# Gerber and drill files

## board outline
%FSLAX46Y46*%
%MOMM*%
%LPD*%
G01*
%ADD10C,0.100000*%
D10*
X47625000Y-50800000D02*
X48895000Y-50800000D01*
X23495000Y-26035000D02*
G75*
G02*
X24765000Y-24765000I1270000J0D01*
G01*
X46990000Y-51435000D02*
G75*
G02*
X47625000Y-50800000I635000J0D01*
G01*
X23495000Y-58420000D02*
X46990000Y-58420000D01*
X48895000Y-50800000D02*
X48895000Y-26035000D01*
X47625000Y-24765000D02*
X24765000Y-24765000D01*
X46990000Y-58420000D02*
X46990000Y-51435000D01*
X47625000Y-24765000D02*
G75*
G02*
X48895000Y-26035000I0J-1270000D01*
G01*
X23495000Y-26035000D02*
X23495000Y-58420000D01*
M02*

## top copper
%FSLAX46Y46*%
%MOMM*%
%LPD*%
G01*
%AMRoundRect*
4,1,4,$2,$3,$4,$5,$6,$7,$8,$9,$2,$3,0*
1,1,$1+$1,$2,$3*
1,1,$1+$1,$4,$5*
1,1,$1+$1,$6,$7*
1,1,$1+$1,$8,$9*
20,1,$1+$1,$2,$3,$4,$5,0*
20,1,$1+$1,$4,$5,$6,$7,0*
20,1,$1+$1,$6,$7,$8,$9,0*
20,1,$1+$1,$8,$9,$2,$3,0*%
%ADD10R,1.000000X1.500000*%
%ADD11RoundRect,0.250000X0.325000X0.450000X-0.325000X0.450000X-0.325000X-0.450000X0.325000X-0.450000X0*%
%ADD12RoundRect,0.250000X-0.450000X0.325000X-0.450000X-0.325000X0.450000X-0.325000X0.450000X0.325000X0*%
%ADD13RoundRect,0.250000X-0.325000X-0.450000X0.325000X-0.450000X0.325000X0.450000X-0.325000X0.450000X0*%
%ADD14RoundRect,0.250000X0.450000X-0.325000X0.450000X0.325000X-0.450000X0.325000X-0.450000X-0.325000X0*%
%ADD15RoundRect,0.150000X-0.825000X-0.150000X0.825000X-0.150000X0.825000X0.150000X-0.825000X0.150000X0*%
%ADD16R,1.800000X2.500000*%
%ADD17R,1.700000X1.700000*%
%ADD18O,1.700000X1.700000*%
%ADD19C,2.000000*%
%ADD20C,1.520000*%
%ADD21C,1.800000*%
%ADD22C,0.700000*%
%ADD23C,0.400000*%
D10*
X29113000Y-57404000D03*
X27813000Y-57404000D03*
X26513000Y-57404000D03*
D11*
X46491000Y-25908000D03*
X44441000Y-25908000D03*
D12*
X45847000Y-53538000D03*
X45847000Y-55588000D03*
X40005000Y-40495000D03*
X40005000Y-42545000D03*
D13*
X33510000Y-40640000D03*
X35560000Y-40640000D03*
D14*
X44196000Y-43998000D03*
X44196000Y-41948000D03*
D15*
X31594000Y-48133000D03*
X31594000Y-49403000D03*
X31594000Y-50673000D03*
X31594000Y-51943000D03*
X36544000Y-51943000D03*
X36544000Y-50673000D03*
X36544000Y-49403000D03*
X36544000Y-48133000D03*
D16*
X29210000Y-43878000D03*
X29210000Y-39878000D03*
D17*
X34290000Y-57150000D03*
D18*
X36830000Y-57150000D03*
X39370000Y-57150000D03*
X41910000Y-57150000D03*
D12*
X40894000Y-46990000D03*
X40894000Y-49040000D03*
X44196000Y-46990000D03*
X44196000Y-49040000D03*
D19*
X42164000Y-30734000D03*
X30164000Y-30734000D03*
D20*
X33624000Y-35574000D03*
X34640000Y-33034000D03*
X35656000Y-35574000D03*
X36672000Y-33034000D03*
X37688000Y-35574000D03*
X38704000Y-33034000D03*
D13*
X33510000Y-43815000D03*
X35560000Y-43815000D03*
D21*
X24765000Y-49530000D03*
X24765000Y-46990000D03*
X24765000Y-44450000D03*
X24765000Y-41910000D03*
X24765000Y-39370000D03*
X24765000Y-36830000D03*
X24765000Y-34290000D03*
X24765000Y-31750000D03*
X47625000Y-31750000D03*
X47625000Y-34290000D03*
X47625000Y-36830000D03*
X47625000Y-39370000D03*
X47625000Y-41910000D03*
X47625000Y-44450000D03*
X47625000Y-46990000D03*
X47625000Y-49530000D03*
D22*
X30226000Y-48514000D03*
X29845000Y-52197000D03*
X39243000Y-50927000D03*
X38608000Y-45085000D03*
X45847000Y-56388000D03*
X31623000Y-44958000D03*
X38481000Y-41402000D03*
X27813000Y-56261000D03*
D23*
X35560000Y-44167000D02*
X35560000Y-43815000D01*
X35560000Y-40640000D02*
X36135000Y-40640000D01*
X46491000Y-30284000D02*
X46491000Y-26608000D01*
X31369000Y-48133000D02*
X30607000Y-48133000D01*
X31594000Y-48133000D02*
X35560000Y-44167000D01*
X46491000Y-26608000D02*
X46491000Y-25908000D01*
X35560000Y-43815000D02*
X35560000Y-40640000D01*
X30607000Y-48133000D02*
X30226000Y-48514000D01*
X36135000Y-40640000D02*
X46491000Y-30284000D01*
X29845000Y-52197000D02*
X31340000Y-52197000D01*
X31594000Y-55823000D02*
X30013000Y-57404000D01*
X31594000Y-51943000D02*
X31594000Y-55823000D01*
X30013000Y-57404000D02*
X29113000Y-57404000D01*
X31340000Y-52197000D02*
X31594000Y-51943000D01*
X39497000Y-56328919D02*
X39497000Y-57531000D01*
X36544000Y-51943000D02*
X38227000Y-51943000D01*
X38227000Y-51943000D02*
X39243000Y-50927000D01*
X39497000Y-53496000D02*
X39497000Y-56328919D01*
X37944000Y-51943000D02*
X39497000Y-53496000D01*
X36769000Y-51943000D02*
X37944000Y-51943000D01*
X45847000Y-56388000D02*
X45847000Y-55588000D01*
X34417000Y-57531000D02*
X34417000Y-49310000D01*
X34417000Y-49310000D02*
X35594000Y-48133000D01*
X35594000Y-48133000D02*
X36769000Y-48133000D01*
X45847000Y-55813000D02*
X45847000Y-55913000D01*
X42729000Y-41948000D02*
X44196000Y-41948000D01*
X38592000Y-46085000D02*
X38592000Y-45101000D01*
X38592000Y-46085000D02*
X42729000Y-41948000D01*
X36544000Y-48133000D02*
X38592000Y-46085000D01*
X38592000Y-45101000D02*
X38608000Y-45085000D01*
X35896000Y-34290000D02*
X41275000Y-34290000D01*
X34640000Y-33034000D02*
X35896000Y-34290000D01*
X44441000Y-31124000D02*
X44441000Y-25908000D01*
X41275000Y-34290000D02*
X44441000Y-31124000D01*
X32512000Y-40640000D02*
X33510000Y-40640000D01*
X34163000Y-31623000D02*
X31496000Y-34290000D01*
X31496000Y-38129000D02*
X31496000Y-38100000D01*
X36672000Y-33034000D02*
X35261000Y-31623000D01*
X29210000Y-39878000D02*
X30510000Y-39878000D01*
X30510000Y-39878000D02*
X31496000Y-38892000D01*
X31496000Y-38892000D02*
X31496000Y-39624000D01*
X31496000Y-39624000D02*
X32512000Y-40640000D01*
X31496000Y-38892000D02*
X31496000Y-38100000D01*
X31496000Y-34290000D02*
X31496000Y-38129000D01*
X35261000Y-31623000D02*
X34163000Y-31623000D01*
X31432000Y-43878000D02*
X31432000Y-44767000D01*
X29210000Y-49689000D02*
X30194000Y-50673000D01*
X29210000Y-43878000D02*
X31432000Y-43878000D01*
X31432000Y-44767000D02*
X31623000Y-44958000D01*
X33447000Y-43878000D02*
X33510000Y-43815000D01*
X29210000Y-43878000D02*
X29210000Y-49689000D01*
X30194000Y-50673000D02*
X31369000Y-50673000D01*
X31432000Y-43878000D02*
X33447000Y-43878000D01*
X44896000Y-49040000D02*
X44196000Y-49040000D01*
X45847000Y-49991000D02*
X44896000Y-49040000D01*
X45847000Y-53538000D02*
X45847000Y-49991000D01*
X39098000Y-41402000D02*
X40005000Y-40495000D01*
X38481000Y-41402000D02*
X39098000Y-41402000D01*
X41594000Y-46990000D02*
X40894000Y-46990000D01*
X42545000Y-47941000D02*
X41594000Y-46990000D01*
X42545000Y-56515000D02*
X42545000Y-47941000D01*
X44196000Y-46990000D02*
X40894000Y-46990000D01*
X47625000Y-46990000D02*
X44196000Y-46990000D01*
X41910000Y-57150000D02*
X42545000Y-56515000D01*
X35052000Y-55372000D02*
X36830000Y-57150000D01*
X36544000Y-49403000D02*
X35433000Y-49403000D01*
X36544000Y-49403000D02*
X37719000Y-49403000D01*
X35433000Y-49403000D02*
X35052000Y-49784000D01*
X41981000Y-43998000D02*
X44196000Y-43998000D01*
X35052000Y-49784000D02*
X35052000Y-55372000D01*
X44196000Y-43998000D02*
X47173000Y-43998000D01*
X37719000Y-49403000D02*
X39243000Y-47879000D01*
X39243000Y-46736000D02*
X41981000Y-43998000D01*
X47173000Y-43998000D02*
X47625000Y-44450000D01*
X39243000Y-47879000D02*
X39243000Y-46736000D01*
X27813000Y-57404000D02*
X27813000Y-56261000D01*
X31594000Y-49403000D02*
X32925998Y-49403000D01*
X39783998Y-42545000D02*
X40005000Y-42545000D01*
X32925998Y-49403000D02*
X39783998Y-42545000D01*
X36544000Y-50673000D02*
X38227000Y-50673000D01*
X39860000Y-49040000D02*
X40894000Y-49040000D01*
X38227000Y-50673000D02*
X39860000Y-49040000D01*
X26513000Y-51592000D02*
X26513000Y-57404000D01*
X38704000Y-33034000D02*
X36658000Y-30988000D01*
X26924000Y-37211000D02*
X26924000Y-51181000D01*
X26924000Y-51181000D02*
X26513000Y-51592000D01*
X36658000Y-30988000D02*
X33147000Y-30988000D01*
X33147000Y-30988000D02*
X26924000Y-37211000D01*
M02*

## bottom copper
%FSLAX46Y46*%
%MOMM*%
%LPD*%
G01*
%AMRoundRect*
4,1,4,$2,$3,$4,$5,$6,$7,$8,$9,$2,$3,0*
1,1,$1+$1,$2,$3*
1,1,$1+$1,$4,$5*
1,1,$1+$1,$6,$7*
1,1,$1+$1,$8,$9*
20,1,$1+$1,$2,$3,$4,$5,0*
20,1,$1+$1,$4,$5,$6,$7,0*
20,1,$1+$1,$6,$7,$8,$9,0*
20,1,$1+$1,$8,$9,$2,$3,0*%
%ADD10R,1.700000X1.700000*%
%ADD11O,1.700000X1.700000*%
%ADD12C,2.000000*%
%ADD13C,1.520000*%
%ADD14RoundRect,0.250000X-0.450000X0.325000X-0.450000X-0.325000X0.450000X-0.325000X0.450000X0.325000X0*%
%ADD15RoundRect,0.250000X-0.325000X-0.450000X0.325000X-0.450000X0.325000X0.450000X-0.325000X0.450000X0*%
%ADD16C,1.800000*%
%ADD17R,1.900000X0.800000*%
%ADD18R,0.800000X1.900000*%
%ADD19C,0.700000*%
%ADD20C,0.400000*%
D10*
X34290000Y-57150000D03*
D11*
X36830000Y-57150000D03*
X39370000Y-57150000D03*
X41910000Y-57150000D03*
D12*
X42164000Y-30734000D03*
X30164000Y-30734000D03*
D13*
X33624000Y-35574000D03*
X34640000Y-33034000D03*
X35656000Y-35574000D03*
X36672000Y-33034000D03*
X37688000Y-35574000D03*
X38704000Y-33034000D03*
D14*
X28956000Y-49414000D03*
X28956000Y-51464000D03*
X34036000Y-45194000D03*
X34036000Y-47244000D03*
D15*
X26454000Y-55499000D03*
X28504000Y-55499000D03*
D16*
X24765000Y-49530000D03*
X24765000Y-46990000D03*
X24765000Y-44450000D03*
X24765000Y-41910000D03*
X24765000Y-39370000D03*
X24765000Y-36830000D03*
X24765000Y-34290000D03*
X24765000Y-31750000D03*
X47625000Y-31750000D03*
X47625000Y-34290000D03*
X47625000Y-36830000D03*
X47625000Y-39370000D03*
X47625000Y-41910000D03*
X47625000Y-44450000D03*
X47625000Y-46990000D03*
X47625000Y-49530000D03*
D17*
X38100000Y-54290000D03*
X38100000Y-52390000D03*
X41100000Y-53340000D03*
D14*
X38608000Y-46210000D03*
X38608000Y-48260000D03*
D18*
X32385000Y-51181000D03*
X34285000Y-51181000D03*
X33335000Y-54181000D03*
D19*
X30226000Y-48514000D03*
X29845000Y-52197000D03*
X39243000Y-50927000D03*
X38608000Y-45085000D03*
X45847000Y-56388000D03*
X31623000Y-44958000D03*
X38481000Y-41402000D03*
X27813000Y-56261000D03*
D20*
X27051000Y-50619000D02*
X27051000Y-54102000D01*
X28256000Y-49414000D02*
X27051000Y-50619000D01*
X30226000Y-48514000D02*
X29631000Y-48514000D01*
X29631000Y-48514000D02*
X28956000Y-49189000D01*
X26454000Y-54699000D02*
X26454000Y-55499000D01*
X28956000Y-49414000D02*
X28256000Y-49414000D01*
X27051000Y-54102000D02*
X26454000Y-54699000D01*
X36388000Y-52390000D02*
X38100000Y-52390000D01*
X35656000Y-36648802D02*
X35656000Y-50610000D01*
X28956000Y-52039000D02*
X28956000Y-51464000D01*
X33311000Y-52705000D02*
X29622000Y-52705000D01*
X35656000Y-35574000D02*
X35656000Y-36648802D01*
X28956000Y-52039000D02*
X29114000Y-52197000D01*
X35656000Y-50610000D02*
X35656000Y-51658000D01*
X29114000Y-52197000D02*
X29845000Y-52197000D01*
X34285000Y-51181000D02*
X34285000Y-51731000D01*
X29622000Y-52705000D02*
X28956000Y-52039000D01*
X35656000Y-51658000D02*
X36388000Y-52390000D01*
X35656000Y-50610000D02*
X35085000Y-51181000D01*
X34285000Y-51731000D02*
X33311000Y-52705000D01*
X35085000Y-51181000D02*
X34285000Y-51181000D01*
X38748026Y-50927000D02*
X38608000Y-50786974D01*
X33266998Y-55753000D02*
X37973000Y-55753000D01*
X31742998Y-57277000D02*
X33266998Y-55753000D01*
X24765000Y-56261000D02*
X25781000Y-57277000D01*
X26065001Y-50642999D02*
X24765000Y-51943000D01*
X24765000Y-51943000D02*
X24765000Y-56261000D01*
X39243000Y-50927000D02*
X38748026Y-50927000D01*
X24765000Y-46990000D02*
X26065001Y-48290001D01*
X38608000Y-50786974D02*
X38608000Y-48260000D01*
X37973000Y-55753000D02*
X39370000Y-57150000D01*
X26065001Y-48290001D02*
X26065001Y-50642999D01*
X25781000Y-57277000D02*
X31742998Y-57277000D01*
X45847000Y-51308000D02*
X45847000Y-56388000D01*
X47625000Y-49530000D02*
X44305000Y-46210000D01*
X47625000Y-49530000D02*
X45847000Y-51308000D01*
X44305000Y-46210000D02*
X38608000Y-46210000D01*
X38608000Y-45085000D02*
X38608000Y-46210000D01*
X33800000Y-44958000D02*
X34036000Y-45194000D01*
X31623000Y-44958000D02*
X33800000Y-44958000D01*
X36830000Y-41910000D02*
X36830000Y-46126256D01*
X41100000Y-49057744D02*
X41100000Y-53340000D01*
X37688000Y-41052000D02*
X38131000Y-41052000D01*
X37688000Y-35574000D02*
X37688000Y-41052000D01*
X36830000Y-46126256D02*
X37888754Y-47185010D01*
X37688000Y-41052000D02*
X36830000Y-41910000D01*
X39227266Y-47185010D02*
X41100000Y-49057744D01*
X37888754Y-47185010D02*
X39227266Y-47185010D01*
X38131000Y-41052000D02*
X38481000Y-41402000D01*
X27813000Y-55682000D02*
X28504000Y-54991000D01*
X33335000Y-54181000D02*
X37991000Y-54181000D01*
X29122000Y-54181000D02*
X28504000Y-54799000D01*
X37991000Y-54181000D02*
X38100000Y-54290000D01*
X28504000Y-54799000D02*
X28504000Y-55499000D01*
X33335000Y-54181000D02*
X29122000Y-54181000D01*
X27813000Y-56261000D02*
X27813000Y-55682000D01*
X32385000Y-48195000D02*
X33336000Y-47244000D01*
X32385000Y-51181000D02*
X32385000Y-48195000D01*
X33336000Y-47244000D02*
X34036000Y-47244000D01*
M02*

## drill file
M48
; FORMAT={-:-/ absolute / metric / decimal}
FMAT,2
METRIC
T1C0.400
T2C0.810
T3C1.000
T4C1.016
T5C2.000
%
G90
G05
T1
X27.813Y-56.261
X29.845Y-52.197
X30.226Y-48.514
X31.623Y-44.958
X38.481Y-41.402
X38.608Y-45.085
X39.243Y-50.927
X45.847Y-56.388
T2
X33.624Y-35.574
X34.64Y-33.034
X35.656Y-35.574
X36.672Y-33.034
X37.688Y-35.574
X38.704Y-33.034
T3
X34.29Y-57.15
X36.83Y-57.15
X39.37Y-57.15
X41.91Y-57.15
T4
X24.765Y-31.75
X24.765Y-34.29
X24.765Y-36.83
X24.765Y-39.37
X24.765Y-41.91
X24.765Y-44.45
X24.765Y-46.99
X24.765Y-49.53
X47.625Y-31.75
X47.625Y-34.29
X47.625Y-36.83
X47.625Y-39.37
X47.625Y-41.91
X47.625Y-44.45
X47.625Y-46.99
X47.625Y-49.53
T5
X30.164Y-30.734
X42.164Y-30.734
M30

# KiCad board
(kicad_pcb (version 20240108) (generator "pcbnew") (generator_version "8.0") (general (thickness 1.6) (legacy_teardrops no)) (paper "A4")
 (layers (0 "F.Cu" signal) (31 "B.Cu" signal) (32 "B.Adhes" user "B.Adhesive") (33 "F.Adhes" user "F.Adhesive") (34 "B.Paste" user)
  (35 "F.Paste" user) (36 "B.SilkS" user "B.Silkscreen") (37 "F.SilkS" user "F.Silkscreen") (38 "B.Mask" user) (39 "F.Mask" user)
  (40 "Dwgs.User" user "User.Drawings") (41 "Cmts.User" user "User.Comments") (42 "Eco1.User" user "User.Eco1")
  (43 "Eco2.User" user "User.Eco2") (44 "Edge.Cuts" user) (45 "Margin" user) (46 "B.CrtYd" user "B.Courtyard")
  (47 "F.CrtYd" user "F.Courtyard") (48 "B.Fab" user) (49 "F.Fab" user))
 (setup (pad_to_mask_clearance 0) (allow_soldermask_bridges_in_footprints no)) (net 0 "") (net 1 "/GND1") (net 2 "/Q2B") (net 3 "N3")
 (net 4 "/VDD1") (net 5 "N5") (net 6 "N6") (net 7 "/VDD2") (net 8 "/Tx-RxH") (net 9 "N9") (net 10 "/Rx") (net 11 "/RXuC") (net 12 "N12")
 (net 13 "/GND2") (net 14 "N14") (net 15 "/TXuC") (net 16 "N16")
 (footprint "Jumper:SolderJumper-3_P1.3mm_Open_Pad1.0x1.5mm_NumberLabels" (layer "F.Cu") (at 27.813 57.404 180)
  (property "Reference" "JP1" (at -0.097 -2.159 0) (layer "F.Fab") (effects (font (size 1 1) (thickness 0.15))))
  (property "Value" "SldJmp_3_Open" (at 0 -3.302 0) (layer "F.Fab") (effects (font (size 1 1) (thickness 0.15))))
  (pad "1" smd rect (at -1.3 0 180) (size 1 1.5) (layers "F.Cu" "F.Mask") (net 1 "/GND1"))
  (pad "2" smd rect (at 0 0 180) (size 1 1.5) (layers "F.Cu" "F.Mask") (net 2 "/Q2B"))
  (pad "3" smd rect (at 1.3 0 180) (size 1 1.5) (layers "F.Cu" "F.Mask") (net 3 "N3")))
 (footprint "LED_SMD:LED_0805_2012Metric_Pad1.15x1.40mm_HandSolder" (layer "F.Cu") (at 45.466 25.908 180)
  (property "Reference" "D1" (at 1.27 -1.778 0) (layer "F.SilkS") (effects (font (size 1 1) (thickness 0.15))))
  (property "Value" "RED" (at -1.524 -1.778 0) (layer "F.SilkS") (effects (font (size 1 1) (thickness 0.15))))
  (pad "1" smd roundrect (at -1.025 0 180) (size 1.15 1.4) (layers "F.Cu" "F.Paste" "F.Mask") (roundrect_rratio 0.217391) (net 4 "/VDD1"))
  (pad "2" smd roundrect (at 1.025 0 180) (size 1.15 1.4) (layers "F.Cu" "F.Paste" "F.Mask") (roundrect_rratio 0.217391) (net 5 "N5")))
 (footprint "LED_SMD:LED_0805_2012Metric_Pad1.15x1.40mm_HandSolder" (layer "F.Cu") (at 45.847 54.563 -90)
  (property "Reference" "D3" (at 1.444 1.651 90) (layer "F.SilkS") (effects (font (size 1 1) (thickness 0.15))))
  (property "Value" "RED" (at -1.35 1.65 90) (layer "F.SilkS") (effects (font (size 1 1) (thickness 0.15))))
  (pad "1" smd roundrect (at -1.025 0 270) (size 1.15 1.4) (layers "F.Cu" "F.Paste" "F.Mask") (roundrect_rratio 0.217391) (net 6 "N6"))
  (pad "2" smd roundrect (at 1.025 0 270) (size 1.15 1.4) (layers "F.Cu" "F.Paste" "F.Mask") (roundrect_rratio 0.217391) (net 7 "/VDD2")))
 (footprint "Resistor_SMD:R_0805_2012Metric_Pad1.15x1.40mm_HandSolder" (layer "F.Cu") (at 40.005 41.52 -90)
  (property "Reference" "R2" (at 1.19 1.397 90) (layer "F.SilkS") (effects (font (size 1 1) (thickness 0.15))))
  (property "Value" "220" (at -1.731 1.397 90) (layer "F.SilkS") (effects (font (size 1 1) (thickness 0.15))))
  (pad "1" smd roundrect (at -1.025 0 270) (size 1.15 1.4) (layers "F.Cu" "F.Paste" "F.Mask") (roundrect_rratio 0.217391) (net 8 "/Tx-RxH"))
  (pad "2" smd roundrect (at 1.025 0 270) (size 1.15 1.4) (layers "F.Cu" "F.Paste" "F.Mask") (roundrect_rratio 0.217391) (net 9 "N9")))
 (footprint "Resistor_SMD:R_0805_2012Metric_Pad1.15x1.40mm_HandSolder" (layer "F.Cu") (at 34.535 40.64)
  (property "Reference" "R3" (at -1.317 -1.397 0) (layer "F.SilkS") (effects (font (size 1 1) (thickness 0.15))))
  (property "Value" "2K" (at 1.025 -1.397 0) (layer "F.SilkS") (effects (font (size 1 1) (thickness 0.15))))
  (pad "1" smd roundrect (at -1.025 0) (size 1.15 1.4) (layers "F.Cu" "F.Paste" "F.Mask") (roundrect_rratio 0.217391) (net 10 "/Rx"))
  (pad "2" smd roundrect (at 1.025 0) (size 1.15 1.4) (layers "F.Cu" "F.Paste" "F.Mask") (roundrect_rratio 0.217391) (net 4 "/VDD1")))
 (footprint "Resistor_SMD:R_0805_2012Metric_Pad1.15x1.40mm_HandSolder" (layer "F.Cu") (at 44.196 42.973 90)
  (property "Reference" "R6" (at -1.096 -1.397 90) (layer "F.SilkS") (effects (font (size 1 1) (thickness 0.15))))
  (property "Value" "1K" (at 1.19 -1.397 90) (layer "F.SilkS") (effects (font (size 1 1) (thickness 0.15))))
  (pad "1" smd roundrect (at -1.025 0 90) (size 1.15 1.4) (layers "F.Cu" "F.Paste" "F.Mask") (roundrect_rratio 0.217391) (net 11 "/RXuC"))
  (pad "2" smd roundrect (at 1.025 0 90) (size 1.15 1.4) (layers "F.Cu" "F.Paste" "F.Mask") (roundrect_rratio 0.217391) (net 7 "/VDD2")))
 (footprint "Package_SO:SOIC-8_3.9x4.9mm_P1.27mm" (layer "F.Cu") (at 34.069 50.038)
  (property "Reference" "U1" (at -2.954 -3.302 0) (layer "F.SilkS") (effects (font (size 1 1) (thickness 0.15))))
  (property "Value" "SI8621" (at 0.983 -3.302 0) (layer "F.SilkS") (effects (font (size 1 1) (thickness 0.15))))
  (pad "1" smd roundrect (at -2.475 -1.905) (size 1.95 0.6) (layers "F.Cu" "F.Paste" "F.Mask") (roundrect_rratio 0.25) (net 4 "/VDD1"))
  (pad "2" smd roundrect (at -2.475 -0.635) (size 1.95 0.6) (layers "F.Cu" "F.Paste" "F.Mask") (roundrect_rratio 0.25) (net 9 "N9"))
  (pad "3" smd roundrect (at -2.475 0.635) (size 1.95 0.6) (layers "F.Cu" "F.Paste" "F.Mask") (roundrect_rratio 0.25) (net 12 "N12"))
  (pad "4" smd roundrect (at -2.475 1.905) (size 1.95 0.6) (layers "F.Cu" "F.Paste" "F.Mask") (roundrect_rratio 0.25) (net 1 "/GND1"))
  (pad "5" smd roundrect (at 2.475 1.905) (size 1.95 0.6) (layers "F.Cu" "F.Paste" "F.Mask") (roundrect_rratio 0.25) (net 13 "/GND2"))
  (pad "6" smd roundrect (at 2.475 0.635) (size 1.95 0.6) (layers "F.Cu" "F.Paste" "F.Mask") (roundrect_rratio 0.25) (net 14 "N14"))
  (pad "7" smd roundrect (at 2.475 -0.635) (size 1.95 0.6) (layers "F.Cu" "F.Paste" "F.Mask") (roundrect_rratio 0.25) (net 11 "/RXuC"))
  (pad "8" smd roundrect (at 2.475 -1.905) (size 1.95 0.6) (layers "F.Cu" "F.Paste" "F.Mask") (roundrect_rratio 0.25) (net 7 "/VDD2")))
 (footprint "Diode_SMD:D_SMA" (layer "F.Cu") (at 29.21 41.878 90)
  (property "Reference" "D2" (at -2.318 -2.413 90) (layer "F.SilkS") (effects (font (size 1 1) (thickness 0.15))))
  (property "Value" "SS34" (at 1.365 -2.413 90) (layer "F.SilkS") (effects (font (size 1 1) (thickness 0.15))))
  (pad "1" smd rect (at -2 0 90) (size 2.5 1.8) (layers "F.Cu" "F.Paste" "F.Mask") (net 12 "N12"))
  (pad "2" smd rect (at 2 0 90) (size 2.5 1.8) (layers "F.Cu" "F.Paste" "F.Mask") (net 10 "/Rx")))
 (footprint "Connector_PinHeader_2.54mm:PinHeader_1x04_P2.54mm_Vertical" (layer "F.Cu") (at 34.29 57.15 90)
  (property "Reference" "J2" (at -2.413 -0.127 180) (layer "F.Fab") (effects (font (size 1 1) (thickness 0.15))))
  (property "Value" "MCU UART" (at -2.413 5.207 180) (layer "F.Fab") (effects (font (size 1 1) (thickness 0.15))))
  (pad "1" thru_hole rect (at 0 0 90) (size 1.7 1.7) (drill 1) (layers "*.Cu" "*.Mask") (remove_unused_layers no) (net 7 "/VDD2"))
  (pad "2" thru_hole oval (at 0 2.54 90) (size 1.7 1.7) (drill 1) (layers "*.Cu" "*.Mask") (remove_unused_layers no) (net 11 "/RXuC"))
  (pad "3" thru_hole oval (at 0 5.08 90) (size 1.7 1.7) (drill 1) (layers "*.Cu" "*.Mask") (remove_unused_layers no) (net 13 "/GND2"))
  (pad "4" thru_hole oval (at 0 7.62 90) (size 1.7 1.7) (drill 1) (layers "*.Cu" "*.Mask") (remove_unused_layers no) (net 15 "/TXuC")))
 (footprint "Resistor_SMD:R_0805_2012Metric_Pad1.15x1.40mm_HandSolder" (layer "F.Cu") (at 40.894 48.015 -90)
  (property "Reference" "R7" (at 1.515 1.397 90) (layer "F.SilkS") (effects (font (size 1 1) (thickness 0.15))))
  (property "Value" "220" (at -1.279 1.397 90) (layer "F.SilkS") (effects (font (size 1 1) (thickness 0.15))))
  (pad "1" smd roundrect (at -1.025 0 270) (size 1.15 1.4) (layers "F.Cu" "F.Paste" "F.Mask") (roundrect_rratio 0.217391) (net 15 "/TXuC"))
  (pad "2" smd roundrect (at 1.025 0 270) (size 1.15 1.4) (layers "F.Cu" "F.Paste" "F.Mask") (roundrect_rratio 0.217391) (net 14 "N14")))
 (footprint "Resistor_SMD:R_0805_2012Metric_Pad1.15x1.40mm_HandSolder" (layer "F.Cu") (at 44.196 48.015 -90)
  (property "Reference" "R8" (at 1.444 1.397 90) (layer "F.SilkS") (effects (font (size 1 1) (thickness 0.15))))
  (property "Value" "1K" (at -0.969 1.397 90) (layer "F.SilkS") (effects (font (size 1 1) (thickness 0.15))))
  (pad "1" smd roundrect (at -1.025 0 270) (size 1.15 1.4) (layers "F.Cu" "F.Paste" "F.Mask") (roundrect_rratio 0.217391) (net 15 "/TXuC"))
  (pad "2" smd roundrect (at 1.025 0 270) (size 1.15 1.4) (layers "F.Cu" "F.Paste" "F.Mask") (roundrect_rratio 0.217391) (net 6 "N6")))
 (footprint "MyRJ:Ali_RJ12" (layer "F.Cu") (at 36.164 30.734 180)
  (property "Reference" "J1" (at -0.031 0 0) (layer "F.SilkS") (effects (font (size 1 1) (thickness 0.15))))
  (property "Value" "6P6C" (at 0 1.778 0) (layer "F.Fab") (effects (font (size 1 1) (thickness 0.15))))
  (pad "" thru_hole circle (at -6 0 180) (size 2 2) (drill 2) (layers "*.Cu" "*.Mask") (remove_unused_layers no))
  (pad "" thru_hole circle (at 6 0 180) (size 2 2) (drill 2) (layers "*.Cu" "*.Mask") (remove_unused_layers no))
  (pad "1" thru_hole circle (at 2.54 -4.84) (size 1.52 1.52) (drill 0.81) (layers "*.Cu" "*.Mask") (remove_unused_layers no))
  (pad "2" thru_hole circle (at 1.524 -2.3) (size 1.52 1.52) (drill 0.81) (layers "*.Cu" "*.Mask") (remove_unused_layers no) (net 5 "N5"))
  (pad "3" thru_hole circle (at 0.508 -4.84) (size 1.52 1.52) (drill 0.81) (layers "*.Cu" "*.Mask") (remove_unused_layers no)
   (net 1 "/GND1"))
  (pad "4" thru_hole circle (at -0.508 -2.3) (size 1.52 1.52) (drill 0.81) (layers "*.Cu" "*.Mask") (remove_unused_layers no) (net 10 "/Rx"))
  (pad "5" thru_hole circle (at -1.524 -4.84) (size 1.52 1.52) (drill 0.81) (layers "*.Cu" "*.Mask") (remove_unused_layers no)
   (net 8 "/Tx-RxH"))
  (pad "6" thru_hole circle (at -2.54 -2.3) (size 1.52 1.52) (drill 0.81) (layers "*.Cu" "*.Mask") (remove_unused_layers no) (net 3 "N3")))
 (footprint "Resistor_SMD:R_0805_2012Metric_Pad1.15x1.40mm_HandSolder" (layer "F.Cu") (at 34.535 43.815)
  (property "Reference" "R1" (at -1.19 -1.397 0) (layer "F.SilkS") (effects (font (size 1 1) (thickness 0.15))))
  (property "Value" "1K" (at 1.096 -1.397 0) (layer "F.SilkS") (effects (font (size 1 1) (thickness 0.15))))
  (pad "1" smd roundrect (at -1.025 0) (size 1.15 1.4) (layers "F.Cu" "F.Paste" "F.Mask") (roundrect_rratio 0.217391) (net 12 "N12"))
  (pad "2" smd roundrect (at 1.025 0) (size 1.15 1.4) (layers "F.Cu" "F.Paste" "F.Mask") (roundrect_rratio 0.217391) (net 4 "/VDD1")))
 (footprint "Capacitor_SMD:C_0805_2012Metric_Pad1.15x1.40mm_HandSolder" (layer "B.Cu") (at 28.956 50.439 -90)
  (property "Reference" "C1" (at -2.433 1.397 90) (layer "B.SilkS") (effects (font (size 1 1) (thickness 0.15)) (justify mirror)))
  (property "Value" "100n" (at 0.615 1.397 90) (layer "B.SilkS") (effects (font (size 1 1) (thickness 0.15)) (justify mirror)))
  (pad "1" smd roundrect (at -1.025 0 270) (size 1.15 1.4) (layers "B.Cu" "B.Paste" "B.Mask") (roundrect_rratio 0.217391) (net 4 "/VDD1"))
  (pad "2" smd roundrect (at 1.025 0 270) (size 1.15 1.4) (layers "B.Cu" "B.Paste" "B.Mask") (roundrect_rratio 0.217391) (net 1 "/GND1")))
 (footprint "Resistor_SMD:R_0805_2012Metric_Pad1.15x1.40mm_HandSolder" (layer "B.Cu") (at 34.036 46.219 -90)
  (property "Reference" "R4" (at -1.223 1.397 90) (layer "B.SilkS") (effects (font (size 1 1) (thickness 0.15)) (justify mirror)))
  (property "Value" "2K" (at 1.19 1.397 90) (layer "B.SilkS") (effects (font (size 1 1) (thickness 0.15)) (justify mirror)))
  (pad "1" smd roundrect (at -1.025 0 270) (size 1.15 1.4) (layers "B.Cu" "B.Paste" "B.Mask") (roundrect_rratio 0.217391) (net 12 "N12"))
  (pad "2" smd roundrect (at 1.025 0 270) (size 1.15 1.4) (layers "B.Cu" "B.Paste" "B.Mask") (roundrect_rratio 0.217391) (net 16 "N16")))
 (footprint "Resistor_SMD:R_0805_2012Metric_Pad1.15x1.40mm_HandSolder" (layer "B.Cu") (at 27.479 55.499)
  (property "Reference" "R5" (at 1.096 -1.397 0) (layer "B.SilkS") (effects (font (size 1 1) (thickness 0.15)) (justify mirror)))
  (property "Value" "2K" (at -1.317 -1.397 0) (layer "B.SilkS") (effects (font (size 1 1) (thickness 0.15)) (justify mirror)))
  (pad "1" smd roundrect (at -1.025 0) (size 1.15 1.4) (layers "B.Cu" "B.Paste" "B.Mask") (roundrect_rratio 0.217391) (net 4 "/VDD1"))
  (pad "2" smd roundrect (at 1.025 0) (size 1.15 1.4) (layers "B.Cu" "B.Paste" "B.Mask") (roundrect_rratio 0.217391) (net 2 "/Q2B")))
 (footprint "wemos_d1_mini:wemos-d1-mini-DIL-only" (layer "B.Cu") (at 36.195 40.64 90)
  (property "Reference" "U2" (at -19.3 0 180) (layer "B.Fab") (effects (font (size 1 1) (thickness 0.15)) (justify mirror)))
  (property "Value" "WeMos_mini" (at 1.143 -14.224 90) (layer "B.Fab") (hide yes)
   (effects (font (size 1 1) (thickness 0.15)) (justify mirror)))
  (pad "1" thru_hole circle (at -8.89 -11.43 90) (size 1.8 1.8) (drill 1.016) (layers "*.Cu" "*.Mask") (remove_unused_layers no))
  (pad "2" thru_hole circle (at -6.35 -11.43 90) (size 1.8 1.8) (drill 1.016) (layers "*.Cu" "*.Mask") (remove_unused_layers no)
   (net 13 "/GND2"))
  (pad "3" thru_hole circle (at -3.81 -11.43 90) (size 1.8 1.8) (drill 1.016) (layers "*.Cu" "*.Mask") (remove_unused_layers no))
  (pad "4" thru_hole circle (at -1.27 -11.43 90) (size 1.8 1.8) (drill 1.016) (layers "*.Cu" "*.Mask") (remove_unused_layers no))
  (pad "5" thru_hole circle (at 1.27 -11.43 90) (size 1.8 1.8) (drill 1.016) (layers "*.Cu" "*.Mask") (remove_unused_layers no))
  (pad "6" thru_hole circle (at 3.81 -11.43 90) (size 1.8 1.8) (drill 1.016) (layers "*.Cu" "*.Mask") (remove_unused_layers no))
  (pad "7" thru_hole circle (at 6.35 -11.43 90) (size 1.8 1.8) (drill 1.016) (layers "*.Cu" "*.Mask") (remove_unused_layers no))
  (pad "8" thru_hole circle (at 8.89 -11.43 90) (size 1.8 1.8) (drill 1.016) (layers "*.Cu" "*.Mask") (remove_unused_layers no))
  (pad "9" thru_hole circle (at 8.89 11.43 90) (size 1.8 1.8) (drill 1.016) (layers "*.Cu" "*.Mask") (remove_unused_layers no))
  (pad "10" thru_hole circle (at 6.35 11.43 90) (size 1.8 1.8) (drill 1.016) (layers "*.Cu" "*.Mask") (remove_unused_layers no))
  (pad "11" thru_hole circle (at 3.81 11.43 90) (size 1.8 1.8) (drill 1.016) (layers "*.Cu" "*.Mask") (remove_unused_layers no))
  (pad "12" thru_hole circle (at 1.27 11.43 90) (size 1.8 1.8) (drill 1.016) (layers "*.Cu" "*.Mask") (remove_unused_layers no))
  (pad "13" thru_hole circle (at -1.27 11.43 90) (size 1.8 1.8) (drill 1.016) (layers "*.Cu" "*.Mask") (remove_unused_layers no))
  (pad "14" thru_hole circle (at -3.81 11.43 90) (size 1.8 1.8) (drill 1.016) (layers "*.Cu" "*.Mask") (remove_unused_layers no)
   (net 11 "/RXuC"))
  (pad "15" thru_hole circle (at -6.35 11.43 90) (size 1.8 1.8) (drill 1.016) (layers "*.Cu" "*.Mask") (remove_unused_layers no)
   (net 15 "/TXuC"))
  (pad "16" thru_hole circle (at -8.89 11.43 90) (size 1.8 1.8) (drill 1.016) (layers "*.Cu" "*.Mask") (remove_unused_layers no)
   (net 7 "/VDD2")))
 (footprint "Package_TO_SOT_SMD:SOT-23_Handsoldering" (layer "B.Cu") (at 39.6 53.34)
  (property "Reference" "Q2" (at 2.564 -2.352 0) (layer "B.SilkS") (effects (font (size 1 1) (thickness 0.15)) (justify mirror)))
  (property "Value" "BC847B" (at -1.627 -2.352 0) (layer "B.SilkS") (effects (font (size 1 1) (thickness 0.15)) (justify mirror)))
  (pad "1" smd rect (at -1.5 0.95) (size 1.9 0.8) (layers "B.Cu" "B.Paste" "B.Mask") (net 2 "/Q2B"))
  (pad "2" smd rect (at -1.5 -0.95) (size 1.9 0.8) (layers "B.Cu" "B.Paste" "B.Mask") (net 1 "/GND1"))
  (pad "3" smd rect (at 1.5 0) (size 1.9 0.8) (layers "B.Cu" "B.Paste" "B.Mask") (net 8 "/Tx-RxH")))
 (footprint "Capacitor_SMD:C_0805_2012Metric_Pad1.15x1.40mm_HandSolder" (layer "B.Cu") (at 38.608 47.235 -90)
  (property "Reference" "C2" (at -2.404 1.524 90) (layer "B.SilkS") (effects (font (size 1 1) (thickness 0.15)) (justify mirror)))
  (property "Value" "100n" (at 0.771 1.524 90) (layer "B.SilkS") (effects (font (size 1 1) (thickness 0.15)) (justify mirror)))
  (pad "1" smd roundrect (at -1.025 0 270) (size 1.15 1.4) (layers "B.Cu" "B.Paste" "B.Mask") (roundrect_rratio 0.217391) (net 7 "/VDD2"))
  (pad "2" smd roundrect (at 1.025 0 270) (size 1.15 1.4) (layers "B.Cu" "B.Paste" "B.Mask") (roundrect_rratio 0.217391) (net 13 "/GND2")))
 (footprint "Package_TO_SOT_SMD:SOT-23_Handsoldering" (layer "B.Cu") (at 33.335 52.681 -90)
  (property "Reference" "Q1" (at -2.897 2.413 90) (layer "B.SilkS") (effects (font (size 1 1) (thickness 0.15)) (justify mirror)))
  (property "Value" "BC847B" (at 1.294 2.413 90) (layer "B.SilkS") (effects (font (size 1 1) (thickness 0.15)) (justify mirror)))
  (pad "1" smd rect (at -1.5 0.95 270) (size 1.9 0.8) (layers "B.Cu" "B.Paste" "B.Mask") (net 16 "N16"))
  (pad "2" smd rect (at -1.5 -0.95 270) (size 1.9 0.8) (layers "B.Cu" "B.Paste" "B.Mask") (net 1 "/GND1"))
  (pad "3" smd rect (at 1.5 0 270) (size 1.9 0.8) (layers "B.Cu" "B.Paste" "B.Mask") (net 2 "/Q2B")))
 (gr_line (start 47.625 50.8) (end 48.895 50.8) (stroke (width 0.1) (type solid)) (layer "Edge.Cuts"))
 (gr_arc (start 23.495 26.035) (mid 23.866974 25.136974) (end 24.765 24.765) (stroke (width 0.1) (type solid)) (layer "Edge.Cuts"))
 (gr_arc (start 46.99 51.435) (mid 47.175987 50.985987) (end 47.625 50.8) (stroke (width 0.1) (type solid)) (layer "Edge.Cuts"))
 (gr_line (start 23.495 58.42) (end 46.99 58.42) (stroke (width 0.1) (type solid)) (layer "Edge.Cuts"))
 (gr_line (start 48.895 50.8) (end 48.895 26.035) (stroke (width 0.1) (type solid)) (layer "Edge.Cuts"))
 (gr_line (start 47.625 24.765) (end 24.765 24.765) (stroke (width 0.1) (type solid)) (layer "Edge.Cuts"))
 (gr_line (start 46.99 58.42) (end 46.99 51.435) (stroke (width 0.1) (type solid)) (layer "Edge.Cuts"))
 (gr_arc (start 47.625 24.765) (mid 48.523026 25.136974) (end 48.895 26.035) (stroke (width 0.1) (type solid)) (layer "Edge.Cuts"))
 (gr_line (start 23.495 26.035) (end 23.495 58.42) (stroke (width 0.1) (type solid)) (layer "Edge.Cuts"))
 (segment (start 35.56 44.167) (end 35.56 43.815) (width 0.4) (layer "F.Cu") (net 4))
 (segment (start 35.56 40.64) (end 36.135 40.64) (width 0.4) (layer "F.Cu") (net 4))
 (segment (start 46.491 30.284) (end 46.491 26.608) (width 0.4) (layer "F.Cu") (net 4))
 (segment (start 31.369 48.133) (end 30.607 48.133) (width 0.4) (layer "F.Cu") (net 4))
 (segment (start 31.594 48.133) (end 35.56 44.167) (width 0.4) (layer "F.Cu") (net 4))
 (segment (start 46.491 26.608) (end 46.491 25.908) (width 0.4) (layer "F.Cu") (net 4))
 (segment (start 35.56 43.815) (end 35.56 40.64) (width 0.4) (layer "F.Cu") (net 4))
 (segment (start 30.607 48.133) (end 30.226 48.514) (width 0.4) (layer "F.Cu") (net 4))
 (segment (start 36.135 40.64) (end 46.491 30.284) (width 0.4) (layer "F.Cu") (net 4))
 (via (at 30.226 48.514) (size 0.7) (drill 0.4) (layers "F.Cu" "B.Cu") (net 4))
 (segment (start 27.051 50.619) (end 27.051 54.102) (width 0.4) (layer "B.Cu") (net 4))
 (segment (start 28.256 49.414) (end 27.051 50.619) (width 0.4) (layer "B.Cu") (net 4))
 (segment (start 30.226 48.514) (end 29.631 48.514) (width 0.4) (layer "B.Cu") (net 4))
 (segment (start 29.631 48.514) (end 28.956 49.189) (width 0.4) (layer "B.Cu") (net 4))
 (segment (start 26.454 54.699) (end 26.454 55.499) (width 0.4) (layer "B.Cu") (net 4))
 (segment (start 28.956 49.414) (end 28.256 49.414) (width 0.4) (layer "B.Cu") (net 4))
 (segment (start 27.051 54.102) (end 26.454 54.699) (width 0.4) (layer "B.Cu") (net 4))
 (segment (start 29.845 52.197) (end 31.34 52.197) (width 0.4) (layer "F.Cu") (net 1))
 (segment (start 31.594 55.823) (end 30.013 57.404) (width 0.4) (layer "F.Cu") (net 1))
 (segment (start 31.594 51.943) (end 31.594 55.823) (width 0.4) (layer "F.Cu") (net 1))
 (segment (start 30.013 57.404) (end 29.113 57.404) (width 0.4) (layer "F.Cu") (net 1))
 (segment (start 31.34 52.197) (end 31.594 51.943) (width 0.4) (layer "F.Cu") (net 1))
 (via (at 29.845 52.197) (size 0.7) (drill 0.4) (layers "F.Cu" "B.Cu") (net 1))
 (segment (start 36.388 52.39) (end 38.1 52.39) (width 0.4) (layer "B.Cu") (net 1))
 (segment (start 35.656 36.648802) (end 35.656 50.61) (width 0.4) (layer "B.Cu") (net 1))
 (segment (start 28.956 52.039) (end 28.956 51.464) (width 0.4) (layer "B.Cu") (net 1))
 (segment (start 33.311 52.705) (end 29.622 52.705) (width 0.4) (layer "B.Cu") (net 1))
 (segment (start 35.656 35.574) (end 35.656 36.648802) (width 0.4) (layer "B.Cu") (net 1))
 (segment (start 28.956 52.039) (end 29.114 52.197) (width 0.4) (layer "B.Cu") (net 1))
 (segment (start 35.656 50.61) (end 35.656 51.658) (width 0.4) (layer "B.Cu") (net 1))
 (segment (start 29.114 52.197) (end 29.845 52.197) (width 0.4) (layer "B.Cu") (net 1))
 (segment (start 34.285 51.181) (end 34.285 51.731) (width 0.4) (layer "B.Cu") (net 1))
 (segment (start 29.622 52.705) (end 28.956 52.039) (width 0.4) (layer "B.Cu") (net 1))
 (segment (start 35.656 51.658) (end 36.388 52.39) (width 0.4) (layer "B.Cu") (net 1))
 (segment (start 35.656 50.61) (end 35.085 51.181) (width 0.4) (layer "B.Cu") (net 1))
 (segment (start 34.285 51.731) (end 33.311 52.705) (width 0.4) (layer "B.Cu") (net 1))
 (segment (start 35.085 51.181) (end 34.285 51.181) (width 0.4) (layer "B.Cu") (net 1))
 (segment (start 39.497 56.328919) (end 39.497 57.531) (width 0.4) (layer "F.Cu") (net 13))
 (segment (start 36.544 51.943) (end 38.227 51.943) (width 0.4) (layer "F.Cu") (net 13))
 (segment (start 38.227 51.943) (end 39.243 50.927) (width 0.4) (layer "F.Cu") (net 13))
 (segment (start 39.497 53.496) (end 39.497 56.328919) (width 0.4) (layer "F.Cu") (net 13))
 (segment (start 37.944 51.943) (end 39.497 53.496) (width 0.4) (layer "F.Cu") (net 13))
 (segment (start 36.769 51.943) (end 37.944 51.943) (width 0.4) (layer "F.Cu") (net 13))
 (via (at 39.243 50.927) (size 0.7) (drill 0.4) (layers "F.Cu" "B.Cu") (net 13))
 (segment (start 38.748026 50.927) (end 38.608 50.786974) (width 0.4) (layer "B.Cu") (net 13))
 (segment (start 33.266998 55.753) (end 37.973 55.753) (width 0.4) (layer "B.Cu") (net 13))
 (segment (start 31.742998 57.277) (end 33.266998 55.753) (width 0.4) (layer "B.Cu") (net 13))
 (segment (start 24.765 56.261) (end 25.781 57.277) (width 0.4) (layer "B.Cu") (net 13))
 (segment (start 26.065001 50.642999) (end 24.765 51.943) (width 0.4) (layer "B.Cu") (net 13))
 (segment (start 24.765 51.943) (end 24.765 56.261) (width 0.4) (layer "B.Cu") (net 13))
 (segment (start 39.243 50.927) (end 38.748026 50.927) (width 0.4) (layer "B.Cu") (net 13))
 (segment (start 24.765 46.99) (end 26.065001 48.290001) (width 0.4) (layer "B.Cu") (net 13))
 (segment (start 38.608 50.786974) (end 38.608 48.26) (width 0.4) (layer "B.Cu") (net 13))
 (segment (start 37.973 55.753) (end 39.37 57.15) (width 0.4) (layer "B.Cu") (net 13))
 (segment (start 26.065001 48.290001) (end 26.065001 50.642999) (width 0.4) (layer "B.Cu") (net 13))
 (segment (start 25.781 57.277) (end 31.742998 57.277) (width 0.4) (layer "B.Cu") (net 13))
 (segment (start 45.847 56.388) (end 45.847 55.588) (width 0.4) (layer "F.Cu") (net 7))
 (segment (start 34.417 57.531) (end 34.417 49.31) (width 0.4) (layer "F.Cu") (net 7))
 (segment (start 34.417 49.31) (end 35.594 48.133) (width 0.4) (layer "F.Cu") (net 7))
 (segment (start 35.594 48.133) (end 36.769 48.133) (width 0.4) (layer "F.Cu") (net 7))
 (segment (start 45.847 55.813) (end 45.847 55.913) (width 0.4) (layer "F.Cu") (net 7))
 (segment (start 42.729 41.948) (end 44.196 41.948) (width 0.4) (layer "F.Cu") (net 7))
 (segment (start 38.592 46.085) (end 38.592 45.101) (width 0.4) (layer "F.Cu") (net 7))
 (segment (start 38.592 46.085) (end 42.729 41.948) (width 0.4) (layer "F.Cu") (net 7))
 (segment (start 36.544 48.133) (end 38.592 46.085) (width 0.4) (layer "F.Cu") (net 7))
 (segment (start 38.592 45.101) (end 38.608 45.085) (width 0.4) (layer "F.Cu") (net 7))
 (via (at 38.608 45.085) (size 0.7) (drill 0.4) (layers "F.Cu" "B.Cu") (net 7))
 (via (at 45.847 56.388) (size 0.7) (drill 0.4) (layers "F.Cu" "B.Cu") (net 7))
 (segment (start 45.847 51.308) (end 45.847 56.388) (width 0.4) (layer "B.Cu") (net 7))
 (segment (start 47.625 49.53) (end 44.305 46.21) (width 0.4) (layer "B.Cu") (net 7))
 (segment (start 47.625 49.53) (end 45.847 51.308) (width 0.4) (layer "B.Cu") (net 7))
 (segment (start 44.305 46.21) (end 38.608 46.21) (width 0.4) (layer "B.Cu") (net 7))
 (segment (start 38.608 45.085) (end 38.608 46.21) (width 0.4) (layer "B.Cu") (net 7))
 (segment (start 35.896 34.29) (end 41.275 34.29) (width 0.4) (layer "F.Cu") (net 5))
 (segment (start 34.64 33.034) (end 35.896 34.29) (width 0.4) (layer "F.Cu") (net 5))
 (segment (start 44.441 31.124) (end 44.441 25.908) (width 0.4) (layer "F.Cu") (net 5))
 (segment (start 41.275 34.29) (end 44.441 31.124) (width 0.4) (layer "F.Cu") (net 5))
 (segment (start 32.512 40.64) (end 33.51 40.64) (width 0.4) (layer "F.Cu") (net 10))
 (segment (start 34.163 31.623) (end 31.496 34.29) (width 0.4) (layer "F.Cu") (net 10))
 (segment (start 31.496 38.129) (end 31.496 38.1) (width 0.4) (layer "F.Cu") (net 10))
 (segment (start 36.672 33.034) (end 35.261 31.623) (width 0.4) (layer "F.Cu") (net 10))
 (segment (start 29.21 39.878) (end 30.51 39.878) (width 0.4) (layer "F.Cu") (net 10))
 (segment (start 30.51 39.878) (end 31.496 38.892) (width 0.4) (layer "F.Cu") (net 10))
 (segment (start 31.496 38.892) (end 31.496 39.624) (width 0.4) (layer "F.Cu") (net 10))
 (segment (start 31.496 39.624) (end 32.512 40.64) (width 0.4) (layer "F.Cu") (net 10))
 (segment (start 31.496 38.892) (end 31.496 38.1) (width 0.4) (layer "F.Cu") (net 10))
 (segment (start 31.496 34.29) (end 31.496 38.129) (width 0.4) (layer "F.Cu") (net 10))
 (segment (start 35.261 31.623) (end 34.163 31.623) (width 0.4) (layer "F.Cu") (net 10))
 (segment (start 31.432 43.878) (end 31.432 44.767) (width 0.4) (layer "F.Cu") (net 12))
 (segment (start 29.21 49.689) (end 30.194 50.673) (width 0.4) (layer "F.Cu") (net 12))
 (segment (start 29.21 43.878) (end 31.432 43.878) (width 0.4) (layer "F.Cu") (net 12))
 (segment (start 31.432 44.767) (end 31.623 44.958) (width 0.4) (layer "F.Cu") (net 12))
 (segment (start 33.447 43.878) (end 33.51 43.815) (width 0.4) (layer "F.Cu") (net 12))
 (segment (start 29.21 43.878) (end 29.21 49.689) (width 0.4) (layer "F.Cu") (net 12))
 (segment (start 30.194 50.673) (end 31.369 50.673) (width 0.4) (layer "F.Cu") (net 12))
 (segment (start 31.432 43.878) (end 33.447 43.878) (width 0.4) (layer "F.Cu") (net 12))
 (via (at 31.623 44.958) (size 0.7) (drill 0.4) (layers "F.Cu" "B.Cu") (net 12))
 (segment (start 33.8 44.958) (end 34.036 45.194) (width 0.4) (layer "B.Cu") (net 12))
 (segment (start 31.623 44.958) (end 33.8 44.958) (width 0.4) (layer "B.Cu") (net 12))
 (segment (start 44.896 49.04) (end 44.196 49.04) (width 0.4) (layer "F.Cu") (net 6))
 (segment (start 45.847 49.991) (end 44.896 49.04) (width 0.4) (layer "F.Cu") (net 6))
 (segment (start 45.847 53.538) (end 45.847 49.991) (width 0.4) (layer "F.Cu") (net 6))
 (segment (start 39.098 41.402) (end 40.005 40.495) (width 0.4) (layer "F.Cu") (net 8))
 (segment (start 38.481 41.402) (end 39.098 41.402) (width 0.4) (layer "F.Cu") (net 8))
 (via (at 38.481 41.402) (size 0.7) (drill 0.4) (layers "F.Cu" "B.Cu") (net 8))
 (segment (start 36.83 41.91) (end 36.83 46.126256) (width 0.4) (layer "B.Cu") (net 8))
 (segment (start 41.1 49.057744) (end 41.1 53.34) (width 0.4) (layer "B.Cu") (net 8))
 (segment (start 37.688 41.052) (end 38.131 41.052) (width 0.4) (layer "B.Cu") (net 8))
 (segment (start 37.688 35.574) (end 37.688 41.052) (width 0.4) (layer "B.Cu") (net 8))
 (segment (start 36.83 46.126256) (end 37.888754 47.18501) (width 0.4) (layer "B.Cu") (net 8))
 (segment (start 37.688 41.052) (end 36.83 41.91) (width 0.4) (layer "B.Cu") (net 8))
 (segment (start 39.227266 47.18501) (end 41.1 49.057744) (width 0.4) (layer "B.Cu") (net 8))
 (segment (start 37.888754 47.18501) (end 39.227266 47.18501) (width 0.4) (layer "B.Cu") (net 8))
 (segment (start 38.131 41.052) (end 38.481 41.402) (width 0.4) (layer "B.Cu") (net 8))
 (segment (start 41.594 46.99) (end 40.894 46.99) (width 0.4) (layer "F.Cu") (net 15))
 (segment (start 42.545 47.941) (end 41.594 46.99) (width 0.4) (layer "F.Cu") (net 15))
 (segment (start 42.545 56.515) (end 42.545 47.941) (width 0.4) (layer "F.Cu") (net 15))
 (segment (start 44.196 46.99) (end 40.894 46.99) (width 0.4) (layer "F.Cu") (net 15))
 (segment (start 47.625 46.99) (end 44.196 46.99) (width 0.4) (layer "F.Cu") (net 15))
 (segment (start 41.91 57.15) (end 42.545 56.515) (width 0.4) (layer "F.Cu") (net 15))
 (segment (start 35.052 55.372) (end 36.83 57.15) (width 0.4) (layer "F.Cu") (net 11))
 (segment (start 36.544 49.403) (end 35.433 49.403) (width 0.4) (layer "F.Cu") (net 11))
 (segment (start 36.544 49.403) (end 37.719 49.403) (width 0.4) (layer "F.Cu") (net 11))
 (segment (start 35.433 49.403) (end 35.052 49.784) (width 0.4) (layer "F.Cu") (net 11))
 (segment (start 41.981 43.998) (end 44.196 43.998) (width 0.4) (layer "F.Cu") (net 11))
 (segment (start 35.052 49.784) (end 35.052 55.372) (width 0.4) (layer "F.Cu") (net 11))
 (segment (start 44.196 43.998) (end 47.173 43.998) (width 0.4) (layer "F.Cu") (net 11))
 (segment (start 37.719 49.403) (end 39.243 47.879) (width 0.4) (layer "F.Cu") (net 11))
 (segment (start 39.243 46.736) (end 41.981 43.998) (width 0.4) (layer "F.Cu") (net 11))
 (segment (start 47.173 43.998) (end 47.625 44.45) (width 0.4) (layer "F.Cu") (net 11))
 (segment (start 39.243 47.879) (end 39.243 46.736) (width 0.4) (layer "F.Cu") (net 11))
 (segment (start 27.813 57.404) (end 27.813 56.261) (width 0.4) (layer "F.Cu") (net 2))
 (via (at 27.813 56.261) (size 0.7) (drill 0.4) (layers "F.Cu" "B.Cu") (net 2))
 (segment (start 27.813 55.682) (end 28.504 54.991) (width 0.4) (layer "B.Cu") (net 2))
 (segment (start 33.335 54.181) (end 37.991 54.181) (width 0.4) (layer "B.Cu") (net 2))
 (segment (start 29.122 54.181) (end 28.504 54.799) (width 0.4) (layer "B.Cu") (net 2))
 (segment (start 37.991 54.181) (end 38.1 54.29) (width 0.4) (layer "B.Cu") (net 2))
 (segment (start 28.504 54.799) (end 28.504 55.499) (width 0.4) (layer "B.Cu") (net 2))
 (segment (start 33.335 54.181) (end 29.122 54.181) (width 0.4) (layer "B.Cu") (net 2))
 (segment (start 27.813 56.261) (end 27.813 55.682) (width 0.4) (layer "B.Cu") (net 2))
 (segment (start 32.385 48.195) (end 33.336 47.244) (width 0.4) (layer "B.Cu") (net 16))
 (segment (start 32.385 51.181) (end 32.385 48.195) (width 0.4) (layer "B.Cu") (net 16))
 (segment (start 33.336 47.244) (end 34.036 47.244) (width 0.4) (layer "B.Cu") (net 16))
 (segment (start 31.594 49.403) (end 32.925998 49.403) (width 0.4) (layer "F.Cu") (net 9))
 (segment (start 39.783998 42.545) (end 40.005 42.545) (width 0.4) (layer "F.Cu") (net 9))
 (segment (start 32.925998 49.403) (end 39.783998 42.545) (width 0.4) (layer "F.Cu") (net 9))
 (segment (start 36.544 50.673) (end 38.227 50.673) (width 0.4) (layer "F.Cu") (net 14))
 (segment (start 39.86 49.04) (end 40.894 49.04) (width 0.4) (layer "F.Cu") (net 14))
 (segment (start 38.227 50.673) (end 39.86 49.04) (width 0.4) (layer "F.Cu") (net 14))
 (segment (start 26.513 51.592) (end 26.513 57.404) (width 0.4) (layer "F.Cu") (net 3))
 (segment (start 38.704 33.034) (end 36.658 30.988) (width 0.4) (layer "F.Cu") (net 3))
 (segment (start 26.924 37.211) (end 26.924 51.181) (width 0.4) (layer "F.Cu") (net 3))
 (segment (start 26.924 51.181) (end 26.513 51.592) (width 0.4) (layer "F.Cu") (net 3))
 (segment (start 36.658 30.988) (end 33.147 30.988) (width 0.4) (layer "F.Cu") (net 3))
 (segment (start 33.147 30.988) (end 26.924 37.211) (width 0.4) (layer "F.Cu") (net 3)))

